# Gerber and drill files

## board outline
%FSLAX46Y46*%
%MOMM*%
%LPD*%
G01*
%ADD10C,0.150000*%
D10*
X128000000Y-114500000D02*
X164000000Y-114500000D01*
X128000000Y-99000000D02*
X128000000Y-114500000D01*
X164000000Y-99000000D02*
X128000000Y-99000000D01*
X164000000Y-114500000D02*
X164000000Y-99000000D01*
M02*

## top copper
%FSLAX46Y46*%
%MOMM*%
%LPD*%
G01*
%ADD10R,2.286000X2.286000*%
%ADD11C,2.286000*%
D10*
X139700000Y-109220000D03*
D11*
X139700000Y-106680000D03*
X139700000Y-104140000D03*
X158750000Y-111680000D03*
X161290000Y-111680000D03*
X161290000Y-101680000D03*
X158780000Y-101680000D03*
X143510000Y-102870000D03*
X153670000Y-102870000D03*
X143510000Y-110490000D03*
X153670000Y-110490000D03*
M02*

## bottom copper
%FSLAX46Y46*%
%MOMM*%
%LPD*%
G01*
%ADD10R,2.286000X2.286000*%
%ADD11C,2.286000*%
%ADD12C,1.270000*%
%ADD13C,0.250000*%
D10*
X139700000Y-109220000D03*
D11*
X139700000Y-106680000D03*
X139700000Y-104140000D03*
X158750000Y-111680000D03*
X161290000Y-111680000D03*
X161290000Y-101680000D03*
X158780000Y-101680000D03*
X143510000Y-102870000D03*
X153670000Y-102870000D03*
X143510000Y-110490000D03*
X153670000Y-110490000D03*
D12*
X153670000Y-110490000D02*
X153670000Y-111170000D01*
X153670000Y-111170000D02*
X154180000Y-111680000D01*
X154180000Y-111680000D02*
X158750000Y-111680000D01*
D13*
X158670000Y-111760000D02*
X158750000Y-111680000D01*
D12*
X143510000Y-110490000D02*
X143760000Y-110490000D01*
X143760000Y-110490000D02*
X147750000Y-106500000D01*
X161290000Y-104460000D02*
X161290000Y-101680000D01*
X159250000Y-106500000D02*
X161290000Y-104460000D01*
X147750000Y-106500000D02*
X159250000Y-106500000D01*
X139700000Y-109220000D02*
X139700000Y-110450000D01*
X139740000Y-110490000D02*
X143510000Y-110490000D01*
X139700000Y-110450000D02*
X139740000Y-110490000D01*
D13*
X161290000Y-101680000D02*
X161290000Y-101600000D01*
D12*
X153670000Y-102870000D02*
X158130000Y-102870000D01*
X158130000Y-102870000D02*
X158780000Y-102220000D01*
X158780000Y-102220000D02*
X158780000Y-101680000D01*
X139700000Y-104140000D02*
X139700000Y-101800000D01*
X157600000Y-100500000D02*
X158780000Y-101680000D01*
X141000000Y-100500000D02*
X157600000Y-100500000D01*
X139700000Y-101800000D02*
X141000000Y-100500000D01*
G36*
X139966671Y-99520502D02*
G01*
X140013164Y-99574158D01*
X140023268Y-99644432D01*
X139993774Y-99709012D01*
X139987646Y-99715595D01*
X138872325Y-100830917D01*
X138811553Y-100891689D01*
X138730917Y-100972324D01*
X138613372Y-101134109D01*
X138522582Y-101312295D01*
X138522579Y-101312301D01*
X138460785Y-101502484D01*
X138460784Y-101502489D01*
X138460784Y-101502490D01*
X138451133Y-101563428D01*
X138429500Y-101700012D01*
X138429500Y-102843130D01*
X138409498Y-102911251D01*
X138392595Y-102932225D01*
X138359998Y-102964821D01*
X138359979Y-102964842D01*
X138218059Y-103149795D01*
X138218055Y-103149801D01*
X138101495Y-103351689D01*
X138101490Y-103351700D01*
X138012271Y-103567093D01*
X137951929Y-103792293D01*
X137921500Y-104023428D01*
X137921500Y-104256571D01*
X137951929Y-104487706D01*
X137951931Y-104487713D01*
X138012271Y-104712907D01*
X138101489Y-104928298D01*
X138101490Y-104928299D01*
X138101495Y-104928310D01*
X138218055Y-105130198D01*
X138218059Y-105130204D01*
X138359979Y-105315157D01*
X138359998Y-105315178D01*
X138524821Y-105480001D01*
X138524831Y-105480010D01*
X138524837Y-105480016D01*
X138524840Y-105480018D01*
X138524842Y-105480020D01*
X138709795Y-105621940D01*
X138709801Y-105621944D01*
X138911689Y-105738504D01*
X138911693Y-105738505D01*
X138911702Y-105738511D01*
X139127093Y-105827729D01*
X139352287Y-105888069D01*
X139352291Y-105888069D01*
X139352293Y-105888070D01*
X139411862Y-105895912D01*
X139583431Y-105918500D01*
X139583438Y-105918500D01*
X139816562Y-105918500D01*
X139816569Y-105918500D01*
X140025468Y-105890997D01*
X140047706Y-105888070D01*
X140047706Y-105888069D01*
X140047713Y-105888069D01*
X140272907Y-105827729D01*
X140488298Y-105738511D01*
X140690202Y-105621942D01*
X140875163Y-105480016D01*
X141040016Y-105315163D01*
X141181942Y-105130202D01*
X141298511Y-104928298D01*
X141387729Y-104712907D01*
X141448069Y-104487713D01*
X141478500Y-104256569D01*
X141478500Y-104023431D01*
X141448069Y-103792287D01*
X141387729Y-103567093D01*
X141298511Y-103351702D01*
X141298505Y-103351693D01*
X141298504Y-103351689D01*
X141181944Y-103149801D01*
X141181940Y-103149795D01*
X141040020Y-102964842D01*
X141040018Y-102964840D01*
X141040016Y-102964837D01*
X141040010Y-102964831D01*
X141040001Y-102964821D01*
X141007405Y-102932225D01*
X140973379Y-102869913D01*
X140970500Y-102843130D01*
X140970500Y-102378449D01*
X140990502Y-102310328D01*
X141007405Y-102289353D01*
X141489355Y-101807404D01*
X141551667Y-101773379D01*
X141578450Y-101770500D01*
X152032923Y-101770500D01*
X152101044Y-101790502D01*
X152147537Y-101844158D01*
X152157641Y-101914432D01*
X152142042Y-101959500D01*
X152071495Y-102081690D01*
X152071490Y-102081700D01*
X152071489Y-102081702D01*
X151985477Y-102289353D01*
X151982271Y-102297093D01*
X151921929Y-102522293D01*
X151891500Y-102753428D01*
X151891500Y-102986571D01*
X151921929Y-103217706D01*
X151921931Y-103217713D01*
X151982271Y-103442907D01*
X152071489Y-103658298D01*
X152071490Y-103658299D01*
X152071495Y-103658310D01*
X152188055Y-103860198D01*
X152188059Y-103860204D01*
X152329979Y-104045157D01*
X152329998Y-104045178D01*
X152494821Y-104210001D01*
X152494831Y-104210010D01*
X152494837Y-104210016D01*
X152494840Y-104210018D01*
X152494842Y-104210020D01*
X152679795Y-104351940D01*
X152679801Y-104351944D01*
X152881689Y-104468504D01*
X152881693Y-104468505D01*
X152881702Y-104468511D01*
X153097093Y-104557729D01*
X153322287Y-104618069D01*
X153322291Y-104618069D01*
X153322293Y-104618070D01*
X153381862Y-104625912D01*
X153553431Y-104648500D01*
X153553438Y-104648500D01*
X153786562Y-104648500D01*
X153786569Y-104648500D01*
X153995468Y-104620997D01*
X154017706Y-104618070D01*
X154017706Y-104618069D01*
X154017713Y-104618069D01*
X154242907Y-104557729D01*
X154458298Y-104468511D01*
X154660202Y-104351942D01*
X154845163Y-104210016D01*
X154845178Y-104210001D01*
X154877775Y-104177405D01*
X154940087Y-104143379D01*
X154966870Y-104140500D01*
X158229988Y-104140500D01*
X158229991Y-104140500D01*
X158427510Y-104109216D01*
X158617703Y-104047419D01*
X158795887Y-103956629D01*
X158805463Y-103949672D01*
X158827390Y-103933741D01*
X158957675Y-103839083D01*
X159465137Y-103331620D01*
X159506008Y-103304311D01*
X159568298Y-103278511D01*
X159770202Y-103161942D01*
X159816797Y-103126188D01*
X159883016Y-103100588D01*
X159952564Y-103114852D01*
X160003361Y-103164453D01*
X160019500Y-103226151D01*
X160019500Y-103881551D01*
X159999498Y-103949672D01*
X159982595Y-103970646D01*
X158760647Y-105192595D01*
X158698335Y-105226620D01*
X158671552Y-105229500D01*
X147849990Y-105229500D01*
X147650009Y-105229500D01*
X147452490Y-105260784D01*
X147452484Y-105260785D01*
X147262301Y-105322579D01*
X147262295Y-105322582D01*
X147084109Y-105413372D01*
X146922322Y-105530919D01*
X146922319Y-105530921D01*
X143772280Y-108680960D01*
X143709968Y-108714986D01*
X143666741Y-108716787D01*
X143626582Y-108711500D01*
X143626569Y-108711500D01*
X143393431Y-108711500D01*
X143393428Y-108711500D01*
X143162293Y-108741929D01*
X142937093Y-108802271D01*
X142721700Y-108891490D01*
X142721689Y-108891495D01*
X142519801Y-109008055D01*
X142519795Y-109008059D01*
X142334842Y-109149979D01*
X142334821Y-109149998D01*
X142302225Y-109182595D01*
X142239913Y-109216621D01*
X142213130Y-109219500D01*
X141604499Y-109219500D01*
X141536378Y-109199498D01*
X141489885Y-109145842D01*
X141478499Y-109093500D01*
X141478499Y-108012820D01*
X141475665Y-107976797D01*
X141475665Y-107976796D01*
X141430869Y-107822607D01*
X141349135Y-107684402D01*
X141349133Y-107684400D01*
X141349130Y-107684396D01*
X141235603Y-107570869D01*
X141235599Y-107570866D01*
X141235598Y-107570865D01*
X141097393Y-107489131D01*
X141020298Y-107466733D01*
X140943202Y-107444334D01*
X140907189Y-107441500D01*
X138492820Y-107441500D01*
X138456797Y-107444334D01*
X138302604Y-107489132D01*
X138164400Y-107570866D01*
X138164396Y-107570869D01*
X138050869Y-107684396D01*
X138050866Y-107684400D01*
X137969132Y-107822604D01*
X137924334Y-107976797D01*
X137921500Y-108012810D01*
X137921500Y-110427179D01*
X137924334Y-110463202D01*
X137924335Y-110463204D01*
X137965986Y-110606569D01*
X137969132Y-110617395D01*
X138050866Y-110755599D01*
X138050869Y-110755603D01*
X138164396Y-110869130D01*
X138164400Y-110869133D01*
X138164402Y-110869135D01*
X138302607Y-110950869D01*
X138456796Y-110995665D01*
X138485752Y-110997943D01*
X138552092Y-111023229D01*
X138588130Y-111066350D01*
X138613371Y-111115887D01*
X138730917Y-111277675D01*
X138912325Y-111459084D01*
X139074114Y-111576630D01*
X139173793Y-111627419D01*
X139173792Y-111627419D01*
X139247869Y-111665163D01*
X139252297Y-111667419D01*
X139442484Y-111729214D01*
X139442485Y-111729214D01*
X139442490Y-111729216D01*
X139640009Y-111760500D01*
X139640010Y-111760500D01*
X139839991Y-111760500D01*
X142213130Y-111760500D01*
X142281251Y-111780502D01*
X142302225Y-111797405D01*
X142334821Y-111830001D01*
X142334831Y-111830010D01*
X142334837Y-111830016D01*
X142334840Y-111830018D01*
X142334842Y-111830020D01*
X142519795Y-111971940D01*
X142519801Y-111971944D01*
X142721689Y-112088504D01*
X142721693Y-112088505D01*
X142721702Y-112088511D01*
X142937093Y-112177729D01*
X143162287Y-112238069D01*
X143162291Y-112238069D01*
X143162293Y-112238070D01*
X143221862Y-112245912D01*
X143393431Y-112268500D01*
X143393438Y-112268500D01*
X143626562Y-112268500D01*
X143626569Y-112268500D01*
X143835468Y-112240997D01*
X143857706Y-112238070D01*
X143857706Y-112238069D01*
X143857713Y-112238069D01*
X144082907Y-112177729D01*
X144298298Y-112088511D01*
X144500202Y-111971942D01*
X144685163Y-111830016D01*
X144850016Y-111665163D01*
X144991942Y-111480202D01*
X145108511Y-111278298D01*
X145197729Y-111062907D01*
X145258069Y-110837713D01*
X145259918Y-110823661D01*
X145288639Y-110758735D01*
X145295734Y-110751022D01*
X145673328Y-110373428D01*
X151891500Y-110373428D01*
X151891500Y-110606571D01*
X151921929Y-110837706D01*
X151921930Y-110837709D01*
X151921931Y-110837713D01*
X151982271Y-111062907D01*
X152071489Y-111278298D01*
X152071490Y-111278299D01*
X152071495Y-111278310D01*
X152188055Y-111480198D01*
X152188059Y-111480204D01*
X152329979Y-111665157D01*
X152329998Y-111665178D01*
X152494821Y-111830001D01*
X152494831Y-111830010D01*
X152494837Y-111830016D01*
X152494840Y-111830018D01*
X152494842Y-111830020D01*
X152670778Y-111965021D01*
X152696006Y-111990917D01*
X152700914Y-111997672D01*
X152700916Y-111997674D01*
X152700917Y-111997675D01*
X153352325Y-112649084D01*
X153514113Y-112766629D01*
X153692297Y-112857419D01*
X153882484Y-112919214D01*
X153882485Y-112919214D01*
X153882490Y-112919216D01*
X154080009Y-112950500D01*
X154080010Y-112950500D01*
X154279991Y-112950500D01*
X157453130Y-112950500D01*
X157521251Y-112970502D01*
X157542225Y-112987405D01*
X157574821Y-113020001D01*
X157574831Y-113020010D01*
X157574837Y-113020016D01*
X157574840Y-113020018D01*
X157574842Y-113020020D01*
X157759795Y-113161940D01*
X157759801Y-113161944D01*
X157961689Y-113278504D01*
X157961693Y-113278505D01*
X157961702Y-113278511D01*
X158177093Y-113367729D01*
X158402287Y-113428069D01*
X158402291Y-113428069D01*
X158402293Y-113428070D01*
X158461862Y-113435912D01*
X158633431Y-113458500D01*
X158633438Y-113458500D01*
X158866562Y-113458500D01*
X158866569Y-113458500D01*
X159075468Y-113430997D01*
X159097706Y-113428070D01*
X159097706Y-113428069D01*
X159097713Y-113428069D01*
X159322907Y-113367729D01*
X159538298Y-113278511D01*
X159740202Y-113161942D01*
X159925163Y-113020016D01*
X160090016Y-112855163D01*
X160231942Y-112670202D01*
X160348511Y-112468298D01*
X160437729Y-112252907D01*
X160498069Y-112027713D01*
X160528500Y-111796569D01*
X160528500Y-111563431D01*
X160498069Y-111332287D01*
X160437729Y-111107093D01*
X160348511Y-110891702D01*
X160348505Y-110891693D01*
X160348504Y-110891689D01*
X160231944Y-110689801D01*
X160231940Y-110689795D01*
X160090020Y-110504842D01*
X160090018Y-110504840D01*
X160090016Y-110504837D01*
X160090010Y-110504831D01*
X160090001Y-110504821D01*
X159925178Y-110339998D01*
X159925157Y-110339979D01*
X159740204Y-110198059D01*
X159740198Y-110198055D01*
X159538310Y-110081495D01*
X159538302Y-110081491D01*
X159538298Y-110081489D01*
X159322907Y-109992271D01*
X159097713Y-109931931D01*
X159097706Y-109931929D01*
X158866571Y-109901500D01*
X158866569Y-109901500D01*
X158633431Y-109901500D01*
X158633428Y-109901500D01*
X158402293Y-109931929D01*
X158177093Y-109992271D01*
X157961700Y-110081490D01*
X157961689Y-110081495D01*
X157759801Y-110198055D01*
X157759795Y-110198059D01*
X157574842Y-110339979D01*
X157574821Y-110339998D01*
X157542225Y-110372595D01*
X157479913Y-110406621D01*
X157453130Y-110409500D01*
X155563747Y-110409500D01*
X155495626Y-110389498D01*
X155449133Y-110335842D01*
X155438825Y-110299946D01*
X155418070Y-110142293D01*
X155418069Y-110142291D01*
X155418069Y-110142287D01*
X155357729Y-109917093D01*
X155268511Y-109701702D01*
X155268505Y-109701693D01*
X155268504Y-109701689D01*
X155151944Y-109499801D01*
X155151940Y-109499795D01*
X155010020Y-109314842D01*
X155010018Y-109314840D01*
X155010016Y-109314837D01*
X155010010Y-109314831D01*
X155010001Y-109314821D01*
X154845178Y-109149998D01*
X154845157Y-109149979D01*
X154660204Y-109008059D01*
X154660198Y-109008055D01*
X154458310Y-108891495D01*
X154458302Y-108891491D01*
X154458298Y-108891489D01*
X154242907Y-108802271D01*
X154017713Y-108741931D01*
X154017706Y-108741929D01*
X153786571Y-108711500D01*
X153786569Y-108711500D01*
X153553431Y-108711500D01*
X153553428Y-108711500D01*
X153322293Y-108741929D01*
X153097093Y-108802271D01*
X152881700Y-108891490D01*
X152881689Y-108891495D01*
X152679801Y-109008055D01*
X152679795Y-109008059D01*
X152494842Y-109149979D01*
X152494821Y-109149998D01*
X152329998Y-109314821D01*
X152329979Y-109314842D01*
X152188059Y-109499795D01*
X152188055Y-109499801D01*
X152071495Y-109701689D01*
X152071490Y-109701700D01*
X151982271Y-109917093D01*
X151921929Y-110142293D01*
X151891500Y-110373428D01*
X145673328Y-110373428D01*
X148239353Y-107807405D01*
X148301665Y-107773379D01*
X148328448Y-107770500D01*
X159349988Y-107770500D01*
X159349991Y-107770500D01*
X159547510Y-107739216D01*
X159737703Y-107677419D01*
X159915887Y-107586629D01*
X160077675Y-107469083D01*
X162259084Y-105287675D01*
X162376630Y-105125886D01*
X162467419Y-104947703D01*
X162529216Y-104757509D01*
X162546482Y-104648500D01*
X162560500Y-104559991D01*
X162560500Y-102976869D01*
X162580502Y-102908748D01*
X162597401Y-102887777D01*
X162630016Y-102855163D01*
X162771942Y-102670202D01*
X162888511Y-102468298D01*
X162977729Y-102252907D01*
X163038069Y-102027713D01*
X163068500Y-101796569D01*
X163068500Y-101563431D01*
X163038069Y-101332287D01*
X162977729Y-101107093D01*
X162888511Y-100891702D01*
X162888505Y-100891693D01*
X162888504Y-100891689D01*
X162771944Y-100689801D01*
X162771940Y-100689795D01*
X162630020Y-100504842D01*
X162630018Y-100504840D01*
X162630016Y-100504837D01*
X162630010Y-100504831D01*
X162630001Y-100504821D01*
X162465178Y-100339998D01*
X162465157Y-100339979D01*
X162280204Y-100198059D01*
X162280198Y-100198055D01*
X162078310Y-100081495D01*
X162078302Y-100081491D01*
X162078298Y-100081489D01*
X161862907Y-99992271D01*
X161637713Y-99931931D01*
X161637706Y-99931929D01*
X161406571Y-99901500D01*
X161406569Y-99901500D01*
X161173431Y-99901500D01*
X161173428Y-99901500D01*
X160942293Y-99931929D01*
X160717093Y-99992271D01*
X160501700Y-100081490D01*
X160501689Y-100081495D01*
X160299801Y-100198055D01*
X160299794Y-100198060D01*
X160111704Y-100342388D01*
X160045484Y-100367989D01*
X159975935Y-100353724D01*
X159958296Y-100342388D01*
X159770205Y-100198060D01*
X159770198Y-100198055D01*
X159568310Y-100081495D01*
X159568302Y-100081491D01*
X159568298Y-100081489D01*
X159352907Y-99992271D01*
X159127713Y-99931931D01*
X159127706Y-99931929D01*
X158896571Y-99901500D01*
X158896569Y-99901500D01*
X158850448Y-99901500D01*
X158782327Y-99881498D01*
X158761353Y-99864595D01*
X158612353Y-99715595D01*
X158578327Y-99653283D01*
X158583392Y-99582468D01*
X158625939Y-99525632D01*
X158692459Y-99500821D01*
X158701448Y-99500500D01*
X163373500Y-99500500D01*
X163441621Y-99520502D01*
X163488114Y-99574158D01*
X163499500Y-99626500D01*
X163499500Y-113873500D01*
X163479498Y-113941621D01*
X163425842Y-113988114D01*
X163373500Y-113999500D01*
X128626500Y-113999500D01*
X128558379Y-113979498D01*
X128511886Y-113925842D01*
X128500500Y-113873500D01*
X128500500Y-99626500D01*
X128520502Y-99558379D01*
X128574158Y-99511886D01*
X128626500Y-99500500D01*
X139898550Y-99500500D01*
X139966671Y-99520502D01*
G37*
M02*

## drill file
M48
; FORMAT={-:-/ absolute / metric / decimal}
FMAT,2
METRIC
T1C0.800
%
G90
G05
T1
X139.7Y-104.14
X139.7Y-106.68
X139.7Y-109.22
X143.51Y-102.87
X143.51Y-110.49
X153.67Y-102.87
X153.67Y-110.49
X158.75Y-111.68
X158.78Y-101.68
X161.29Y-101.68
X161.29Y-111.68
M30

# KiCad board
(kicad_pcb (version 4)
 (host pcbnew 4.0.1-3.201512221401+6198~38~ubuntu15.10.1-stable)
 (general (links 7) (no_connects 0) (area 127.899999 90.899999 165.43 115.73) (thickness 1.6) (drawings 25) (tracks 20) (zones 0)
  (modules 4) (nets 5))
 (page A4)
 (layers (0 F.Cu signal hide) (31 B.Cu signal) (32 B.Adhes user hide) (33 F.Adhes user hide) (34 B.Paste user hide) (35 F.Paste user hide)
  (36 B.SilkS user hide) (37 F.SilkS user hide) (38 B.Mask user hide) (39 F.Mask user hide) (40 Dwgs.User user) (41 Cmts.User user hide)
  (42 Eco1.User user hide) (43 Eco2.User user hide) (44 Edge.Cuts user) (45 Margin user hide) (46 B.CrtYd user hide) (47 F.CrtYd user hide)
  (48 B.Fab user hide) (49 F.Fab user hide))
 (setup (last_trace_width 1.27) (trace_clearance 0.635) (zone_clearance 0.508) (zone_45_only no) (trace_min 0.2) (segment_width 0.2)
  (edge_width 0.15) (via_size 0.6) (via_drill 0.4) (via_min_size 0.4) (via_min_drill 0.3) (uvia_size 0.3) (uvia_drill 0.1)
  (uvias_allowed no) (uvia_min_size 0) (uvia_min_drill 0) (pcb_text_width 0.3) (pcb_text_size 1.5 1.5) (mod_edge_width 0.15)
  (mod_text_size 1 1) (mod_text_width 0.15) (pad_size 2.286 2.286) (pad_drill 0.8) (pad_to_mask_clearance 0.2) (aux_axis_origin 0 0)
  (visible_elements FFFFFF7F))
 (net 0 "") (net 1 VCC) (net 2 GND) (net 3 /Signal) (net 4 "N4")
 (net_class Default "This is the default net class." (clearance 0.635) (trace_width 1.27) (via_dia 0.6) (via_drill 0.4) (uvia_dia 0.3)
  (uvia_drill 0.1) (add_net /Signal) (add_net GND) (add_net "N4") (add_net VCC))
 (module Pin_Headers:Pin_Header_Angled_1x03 (layer F.Cu) (at 139.7 109.22 180)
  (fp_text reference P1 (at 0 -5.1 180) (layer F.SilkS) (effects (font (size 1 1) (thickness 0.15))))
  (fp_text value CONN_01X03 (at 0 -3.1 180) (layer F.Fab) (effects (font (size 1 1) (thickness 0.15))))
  (pad 1 thru_hole rect (at 0 0 180) (size 2.286 2.286) (drill 0.8) (layers *.Cu *.Mask F.SilkS) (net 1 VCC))
  (pad 2 thru_hole circle (at 0 2.54 180) (size 2.286 2.286) (drill 0.8) (layers *.Cu *.Mask F.SilkS) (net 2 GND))
  (pad 3 thru_hole circle (at 0 5.08 180) (size 2.286 2.286) (drill 0.8) (layers *.Cu *.Mask F.SilkS) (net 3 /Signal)))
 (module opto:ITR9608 (layer F.Cu) (at 160.02 106.68 90)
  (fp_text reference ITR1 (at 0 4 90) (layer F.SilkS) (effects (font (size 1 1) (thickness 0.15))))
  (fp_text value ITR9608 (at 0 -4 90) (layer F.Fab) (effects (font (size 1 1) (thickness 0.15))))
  (pad 1 thru_hole circle (at -5 -1.27 90) (size 2.286 2.286) (drill 0.8) (layers *.Cu *.Mask F.SilkS) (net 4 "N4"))
  (pad 2 thru_hole circle (at -5 1.27 90) (size 2.286 2.286) (drill 0.8) (layers *.Cu *.Mask F.SilkS) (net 2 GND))
  (pad 4 thru_hole circle (at 5 1.27 90) (size 2.286 2.286) (drill 0.8) (layers *.Cu *.Mask F.SilkS) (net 1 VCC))
  (pad 3 thru_hole circle (at 5 -1.24 90) (size 2.286 2.286) (drill 0.8) (layers *.Cu *.Mask F.SilkS) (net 3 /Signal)))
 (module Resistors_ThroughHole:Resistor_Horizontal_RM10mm (layer F.Cu) (at 148.59 102.87)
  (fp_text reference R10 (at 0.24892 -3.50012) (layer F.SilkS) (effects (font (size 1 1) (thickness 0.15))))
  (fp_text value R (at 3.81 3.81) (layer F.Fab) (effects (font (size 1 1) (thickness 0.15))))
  (pad 1 thru_hole circle (at -5.08 0) (size 2.286 2.286) (drill 0.8) (layers *.Cu *.SilkS *.Mask) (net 2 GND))
  (pad 2 thru_hole circle (at 5.08 0) (size 2.286 2.286) (drill 0.8) (layers *.Cu *.SilkS *.Mask) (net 3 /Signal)))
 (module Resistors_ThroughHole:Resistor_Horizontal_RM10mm (layer F.Cu) (at 148.59 110.49)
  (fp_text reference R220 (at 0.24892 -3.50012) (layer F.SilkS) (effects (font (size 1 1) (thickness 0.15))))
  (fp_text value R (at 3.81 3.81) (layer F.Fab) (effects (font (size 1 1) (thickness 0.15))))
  (pad 1 thru_hole circle (at -5.08 0) (size 2.286 2.286) (drill 0.8) (layers *.Cu *.SilkS *.Mask) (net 1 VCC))
  (pad 2 thru_hole circle (at 5.08 0) (size 2.286 2.286) (drill 0.8) (layers *.Cu *.SilkS *.Mask) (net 4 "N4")))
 (gr_line (start 128 114.5) (end 164 114.5) (angle 90) (layer Edge.Cuts) (width 0.15))
 (gr_line (start 128 99) (end 128 114.5) (angle 90) (layer Edge.Cuts) (width 0.15))
 (gr_line (start 164 99) (end 128 99) (angle 90) (layer Edge.Cuts) (width 0.15))
 (gr_line (start 164 114.5) (end 164 99) (angle 90) (layer Edge.Cuts) (width 0.15))
 (segment (start 153.67 110.49) (end 153.67 111.17) (width 1.27) (layer B.Cu) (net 4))
 (segment (start 153.67 111.17) (end 154.18 111.68) (width 1.27) (layer B.Cu) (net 4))
 (segment (start 154.18 111.68) (end 158.75 111.68) (width 1.27) (layer B.Cu) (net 4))
 (segment (start 158.67 111.76) (end 158.75 111.68) (width 0.25) (layer B.Cu) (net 4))
 (segment (start 143.51 110.49) (end 143.76 110.49) (width 1.27) (layer B.Cu) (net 1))
 (segment (start 143.76 110.49) (end 147.75 106.5) (width 1.27) (layer B.Cu) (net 1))
 (segment (start 161.29 104.46) (end 161.29 101.68) (width 1.27) (layer B.Cu) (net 1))
 (segment (start 159.25 106.5) (end 161.29 104.46) (width 1.27) (layer B.Cu) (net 1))
 (segment (start 147.75 106.5) (end 159.25 106.5) (width 1.27) (layer B.Cu) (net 1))
 (segment (start 139.7 109.22) (end 139.7 110.45) (width 1.27) (layer B.Cu) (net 1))
 (segment (start 139.74 110.49) (end 143.51 110.49) (width 1.27) (layer B.Cu) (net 1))
 (segment (start 139.7 110.45) (end 139.74 110.49) (width 1.27) (layer B.Cu) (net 1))
 (segment (start 161.29 101.68) (end 161.29 101.6) (width 0.25) (layer B.Cu) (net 1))
 (segment (start 153.67 102.87) (end 158.13 102.87) (width 1.27) (layer B.Cu) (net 3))
 (segment (start 158.13 102.87) (end 158.78 102.22) (width 1.27) (layer B.Cu) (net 3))
 (segment (start 158.78 102.22) (end 158.78 101.68) (width 1.27) (layer B.Cu) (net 3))
 (segment (start 139.7 104.14) (end 139.7 101.8) (width 1.27) (layer B.Cu) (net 3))
 (segment (start 157.6 100.5) (end 158.78 101.68) (width 1.27) (layer B.Cu) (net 3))
 (segment (start 141 100.5) (end 157.6 100.5) (width 1.27) (layer B.Cu) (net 3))
 (segment (start 139.7 101.8) (end 141 100.5) (width 1.27) (layer B.Cu) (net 3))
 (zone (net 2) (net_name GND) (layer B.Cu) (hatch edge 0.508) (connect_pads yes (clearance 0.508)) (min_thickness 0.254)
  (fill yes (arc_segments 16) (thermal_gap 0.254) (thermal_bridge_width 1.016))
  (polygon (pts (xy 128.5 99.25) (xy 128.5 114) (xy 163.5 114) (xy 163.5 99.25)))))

